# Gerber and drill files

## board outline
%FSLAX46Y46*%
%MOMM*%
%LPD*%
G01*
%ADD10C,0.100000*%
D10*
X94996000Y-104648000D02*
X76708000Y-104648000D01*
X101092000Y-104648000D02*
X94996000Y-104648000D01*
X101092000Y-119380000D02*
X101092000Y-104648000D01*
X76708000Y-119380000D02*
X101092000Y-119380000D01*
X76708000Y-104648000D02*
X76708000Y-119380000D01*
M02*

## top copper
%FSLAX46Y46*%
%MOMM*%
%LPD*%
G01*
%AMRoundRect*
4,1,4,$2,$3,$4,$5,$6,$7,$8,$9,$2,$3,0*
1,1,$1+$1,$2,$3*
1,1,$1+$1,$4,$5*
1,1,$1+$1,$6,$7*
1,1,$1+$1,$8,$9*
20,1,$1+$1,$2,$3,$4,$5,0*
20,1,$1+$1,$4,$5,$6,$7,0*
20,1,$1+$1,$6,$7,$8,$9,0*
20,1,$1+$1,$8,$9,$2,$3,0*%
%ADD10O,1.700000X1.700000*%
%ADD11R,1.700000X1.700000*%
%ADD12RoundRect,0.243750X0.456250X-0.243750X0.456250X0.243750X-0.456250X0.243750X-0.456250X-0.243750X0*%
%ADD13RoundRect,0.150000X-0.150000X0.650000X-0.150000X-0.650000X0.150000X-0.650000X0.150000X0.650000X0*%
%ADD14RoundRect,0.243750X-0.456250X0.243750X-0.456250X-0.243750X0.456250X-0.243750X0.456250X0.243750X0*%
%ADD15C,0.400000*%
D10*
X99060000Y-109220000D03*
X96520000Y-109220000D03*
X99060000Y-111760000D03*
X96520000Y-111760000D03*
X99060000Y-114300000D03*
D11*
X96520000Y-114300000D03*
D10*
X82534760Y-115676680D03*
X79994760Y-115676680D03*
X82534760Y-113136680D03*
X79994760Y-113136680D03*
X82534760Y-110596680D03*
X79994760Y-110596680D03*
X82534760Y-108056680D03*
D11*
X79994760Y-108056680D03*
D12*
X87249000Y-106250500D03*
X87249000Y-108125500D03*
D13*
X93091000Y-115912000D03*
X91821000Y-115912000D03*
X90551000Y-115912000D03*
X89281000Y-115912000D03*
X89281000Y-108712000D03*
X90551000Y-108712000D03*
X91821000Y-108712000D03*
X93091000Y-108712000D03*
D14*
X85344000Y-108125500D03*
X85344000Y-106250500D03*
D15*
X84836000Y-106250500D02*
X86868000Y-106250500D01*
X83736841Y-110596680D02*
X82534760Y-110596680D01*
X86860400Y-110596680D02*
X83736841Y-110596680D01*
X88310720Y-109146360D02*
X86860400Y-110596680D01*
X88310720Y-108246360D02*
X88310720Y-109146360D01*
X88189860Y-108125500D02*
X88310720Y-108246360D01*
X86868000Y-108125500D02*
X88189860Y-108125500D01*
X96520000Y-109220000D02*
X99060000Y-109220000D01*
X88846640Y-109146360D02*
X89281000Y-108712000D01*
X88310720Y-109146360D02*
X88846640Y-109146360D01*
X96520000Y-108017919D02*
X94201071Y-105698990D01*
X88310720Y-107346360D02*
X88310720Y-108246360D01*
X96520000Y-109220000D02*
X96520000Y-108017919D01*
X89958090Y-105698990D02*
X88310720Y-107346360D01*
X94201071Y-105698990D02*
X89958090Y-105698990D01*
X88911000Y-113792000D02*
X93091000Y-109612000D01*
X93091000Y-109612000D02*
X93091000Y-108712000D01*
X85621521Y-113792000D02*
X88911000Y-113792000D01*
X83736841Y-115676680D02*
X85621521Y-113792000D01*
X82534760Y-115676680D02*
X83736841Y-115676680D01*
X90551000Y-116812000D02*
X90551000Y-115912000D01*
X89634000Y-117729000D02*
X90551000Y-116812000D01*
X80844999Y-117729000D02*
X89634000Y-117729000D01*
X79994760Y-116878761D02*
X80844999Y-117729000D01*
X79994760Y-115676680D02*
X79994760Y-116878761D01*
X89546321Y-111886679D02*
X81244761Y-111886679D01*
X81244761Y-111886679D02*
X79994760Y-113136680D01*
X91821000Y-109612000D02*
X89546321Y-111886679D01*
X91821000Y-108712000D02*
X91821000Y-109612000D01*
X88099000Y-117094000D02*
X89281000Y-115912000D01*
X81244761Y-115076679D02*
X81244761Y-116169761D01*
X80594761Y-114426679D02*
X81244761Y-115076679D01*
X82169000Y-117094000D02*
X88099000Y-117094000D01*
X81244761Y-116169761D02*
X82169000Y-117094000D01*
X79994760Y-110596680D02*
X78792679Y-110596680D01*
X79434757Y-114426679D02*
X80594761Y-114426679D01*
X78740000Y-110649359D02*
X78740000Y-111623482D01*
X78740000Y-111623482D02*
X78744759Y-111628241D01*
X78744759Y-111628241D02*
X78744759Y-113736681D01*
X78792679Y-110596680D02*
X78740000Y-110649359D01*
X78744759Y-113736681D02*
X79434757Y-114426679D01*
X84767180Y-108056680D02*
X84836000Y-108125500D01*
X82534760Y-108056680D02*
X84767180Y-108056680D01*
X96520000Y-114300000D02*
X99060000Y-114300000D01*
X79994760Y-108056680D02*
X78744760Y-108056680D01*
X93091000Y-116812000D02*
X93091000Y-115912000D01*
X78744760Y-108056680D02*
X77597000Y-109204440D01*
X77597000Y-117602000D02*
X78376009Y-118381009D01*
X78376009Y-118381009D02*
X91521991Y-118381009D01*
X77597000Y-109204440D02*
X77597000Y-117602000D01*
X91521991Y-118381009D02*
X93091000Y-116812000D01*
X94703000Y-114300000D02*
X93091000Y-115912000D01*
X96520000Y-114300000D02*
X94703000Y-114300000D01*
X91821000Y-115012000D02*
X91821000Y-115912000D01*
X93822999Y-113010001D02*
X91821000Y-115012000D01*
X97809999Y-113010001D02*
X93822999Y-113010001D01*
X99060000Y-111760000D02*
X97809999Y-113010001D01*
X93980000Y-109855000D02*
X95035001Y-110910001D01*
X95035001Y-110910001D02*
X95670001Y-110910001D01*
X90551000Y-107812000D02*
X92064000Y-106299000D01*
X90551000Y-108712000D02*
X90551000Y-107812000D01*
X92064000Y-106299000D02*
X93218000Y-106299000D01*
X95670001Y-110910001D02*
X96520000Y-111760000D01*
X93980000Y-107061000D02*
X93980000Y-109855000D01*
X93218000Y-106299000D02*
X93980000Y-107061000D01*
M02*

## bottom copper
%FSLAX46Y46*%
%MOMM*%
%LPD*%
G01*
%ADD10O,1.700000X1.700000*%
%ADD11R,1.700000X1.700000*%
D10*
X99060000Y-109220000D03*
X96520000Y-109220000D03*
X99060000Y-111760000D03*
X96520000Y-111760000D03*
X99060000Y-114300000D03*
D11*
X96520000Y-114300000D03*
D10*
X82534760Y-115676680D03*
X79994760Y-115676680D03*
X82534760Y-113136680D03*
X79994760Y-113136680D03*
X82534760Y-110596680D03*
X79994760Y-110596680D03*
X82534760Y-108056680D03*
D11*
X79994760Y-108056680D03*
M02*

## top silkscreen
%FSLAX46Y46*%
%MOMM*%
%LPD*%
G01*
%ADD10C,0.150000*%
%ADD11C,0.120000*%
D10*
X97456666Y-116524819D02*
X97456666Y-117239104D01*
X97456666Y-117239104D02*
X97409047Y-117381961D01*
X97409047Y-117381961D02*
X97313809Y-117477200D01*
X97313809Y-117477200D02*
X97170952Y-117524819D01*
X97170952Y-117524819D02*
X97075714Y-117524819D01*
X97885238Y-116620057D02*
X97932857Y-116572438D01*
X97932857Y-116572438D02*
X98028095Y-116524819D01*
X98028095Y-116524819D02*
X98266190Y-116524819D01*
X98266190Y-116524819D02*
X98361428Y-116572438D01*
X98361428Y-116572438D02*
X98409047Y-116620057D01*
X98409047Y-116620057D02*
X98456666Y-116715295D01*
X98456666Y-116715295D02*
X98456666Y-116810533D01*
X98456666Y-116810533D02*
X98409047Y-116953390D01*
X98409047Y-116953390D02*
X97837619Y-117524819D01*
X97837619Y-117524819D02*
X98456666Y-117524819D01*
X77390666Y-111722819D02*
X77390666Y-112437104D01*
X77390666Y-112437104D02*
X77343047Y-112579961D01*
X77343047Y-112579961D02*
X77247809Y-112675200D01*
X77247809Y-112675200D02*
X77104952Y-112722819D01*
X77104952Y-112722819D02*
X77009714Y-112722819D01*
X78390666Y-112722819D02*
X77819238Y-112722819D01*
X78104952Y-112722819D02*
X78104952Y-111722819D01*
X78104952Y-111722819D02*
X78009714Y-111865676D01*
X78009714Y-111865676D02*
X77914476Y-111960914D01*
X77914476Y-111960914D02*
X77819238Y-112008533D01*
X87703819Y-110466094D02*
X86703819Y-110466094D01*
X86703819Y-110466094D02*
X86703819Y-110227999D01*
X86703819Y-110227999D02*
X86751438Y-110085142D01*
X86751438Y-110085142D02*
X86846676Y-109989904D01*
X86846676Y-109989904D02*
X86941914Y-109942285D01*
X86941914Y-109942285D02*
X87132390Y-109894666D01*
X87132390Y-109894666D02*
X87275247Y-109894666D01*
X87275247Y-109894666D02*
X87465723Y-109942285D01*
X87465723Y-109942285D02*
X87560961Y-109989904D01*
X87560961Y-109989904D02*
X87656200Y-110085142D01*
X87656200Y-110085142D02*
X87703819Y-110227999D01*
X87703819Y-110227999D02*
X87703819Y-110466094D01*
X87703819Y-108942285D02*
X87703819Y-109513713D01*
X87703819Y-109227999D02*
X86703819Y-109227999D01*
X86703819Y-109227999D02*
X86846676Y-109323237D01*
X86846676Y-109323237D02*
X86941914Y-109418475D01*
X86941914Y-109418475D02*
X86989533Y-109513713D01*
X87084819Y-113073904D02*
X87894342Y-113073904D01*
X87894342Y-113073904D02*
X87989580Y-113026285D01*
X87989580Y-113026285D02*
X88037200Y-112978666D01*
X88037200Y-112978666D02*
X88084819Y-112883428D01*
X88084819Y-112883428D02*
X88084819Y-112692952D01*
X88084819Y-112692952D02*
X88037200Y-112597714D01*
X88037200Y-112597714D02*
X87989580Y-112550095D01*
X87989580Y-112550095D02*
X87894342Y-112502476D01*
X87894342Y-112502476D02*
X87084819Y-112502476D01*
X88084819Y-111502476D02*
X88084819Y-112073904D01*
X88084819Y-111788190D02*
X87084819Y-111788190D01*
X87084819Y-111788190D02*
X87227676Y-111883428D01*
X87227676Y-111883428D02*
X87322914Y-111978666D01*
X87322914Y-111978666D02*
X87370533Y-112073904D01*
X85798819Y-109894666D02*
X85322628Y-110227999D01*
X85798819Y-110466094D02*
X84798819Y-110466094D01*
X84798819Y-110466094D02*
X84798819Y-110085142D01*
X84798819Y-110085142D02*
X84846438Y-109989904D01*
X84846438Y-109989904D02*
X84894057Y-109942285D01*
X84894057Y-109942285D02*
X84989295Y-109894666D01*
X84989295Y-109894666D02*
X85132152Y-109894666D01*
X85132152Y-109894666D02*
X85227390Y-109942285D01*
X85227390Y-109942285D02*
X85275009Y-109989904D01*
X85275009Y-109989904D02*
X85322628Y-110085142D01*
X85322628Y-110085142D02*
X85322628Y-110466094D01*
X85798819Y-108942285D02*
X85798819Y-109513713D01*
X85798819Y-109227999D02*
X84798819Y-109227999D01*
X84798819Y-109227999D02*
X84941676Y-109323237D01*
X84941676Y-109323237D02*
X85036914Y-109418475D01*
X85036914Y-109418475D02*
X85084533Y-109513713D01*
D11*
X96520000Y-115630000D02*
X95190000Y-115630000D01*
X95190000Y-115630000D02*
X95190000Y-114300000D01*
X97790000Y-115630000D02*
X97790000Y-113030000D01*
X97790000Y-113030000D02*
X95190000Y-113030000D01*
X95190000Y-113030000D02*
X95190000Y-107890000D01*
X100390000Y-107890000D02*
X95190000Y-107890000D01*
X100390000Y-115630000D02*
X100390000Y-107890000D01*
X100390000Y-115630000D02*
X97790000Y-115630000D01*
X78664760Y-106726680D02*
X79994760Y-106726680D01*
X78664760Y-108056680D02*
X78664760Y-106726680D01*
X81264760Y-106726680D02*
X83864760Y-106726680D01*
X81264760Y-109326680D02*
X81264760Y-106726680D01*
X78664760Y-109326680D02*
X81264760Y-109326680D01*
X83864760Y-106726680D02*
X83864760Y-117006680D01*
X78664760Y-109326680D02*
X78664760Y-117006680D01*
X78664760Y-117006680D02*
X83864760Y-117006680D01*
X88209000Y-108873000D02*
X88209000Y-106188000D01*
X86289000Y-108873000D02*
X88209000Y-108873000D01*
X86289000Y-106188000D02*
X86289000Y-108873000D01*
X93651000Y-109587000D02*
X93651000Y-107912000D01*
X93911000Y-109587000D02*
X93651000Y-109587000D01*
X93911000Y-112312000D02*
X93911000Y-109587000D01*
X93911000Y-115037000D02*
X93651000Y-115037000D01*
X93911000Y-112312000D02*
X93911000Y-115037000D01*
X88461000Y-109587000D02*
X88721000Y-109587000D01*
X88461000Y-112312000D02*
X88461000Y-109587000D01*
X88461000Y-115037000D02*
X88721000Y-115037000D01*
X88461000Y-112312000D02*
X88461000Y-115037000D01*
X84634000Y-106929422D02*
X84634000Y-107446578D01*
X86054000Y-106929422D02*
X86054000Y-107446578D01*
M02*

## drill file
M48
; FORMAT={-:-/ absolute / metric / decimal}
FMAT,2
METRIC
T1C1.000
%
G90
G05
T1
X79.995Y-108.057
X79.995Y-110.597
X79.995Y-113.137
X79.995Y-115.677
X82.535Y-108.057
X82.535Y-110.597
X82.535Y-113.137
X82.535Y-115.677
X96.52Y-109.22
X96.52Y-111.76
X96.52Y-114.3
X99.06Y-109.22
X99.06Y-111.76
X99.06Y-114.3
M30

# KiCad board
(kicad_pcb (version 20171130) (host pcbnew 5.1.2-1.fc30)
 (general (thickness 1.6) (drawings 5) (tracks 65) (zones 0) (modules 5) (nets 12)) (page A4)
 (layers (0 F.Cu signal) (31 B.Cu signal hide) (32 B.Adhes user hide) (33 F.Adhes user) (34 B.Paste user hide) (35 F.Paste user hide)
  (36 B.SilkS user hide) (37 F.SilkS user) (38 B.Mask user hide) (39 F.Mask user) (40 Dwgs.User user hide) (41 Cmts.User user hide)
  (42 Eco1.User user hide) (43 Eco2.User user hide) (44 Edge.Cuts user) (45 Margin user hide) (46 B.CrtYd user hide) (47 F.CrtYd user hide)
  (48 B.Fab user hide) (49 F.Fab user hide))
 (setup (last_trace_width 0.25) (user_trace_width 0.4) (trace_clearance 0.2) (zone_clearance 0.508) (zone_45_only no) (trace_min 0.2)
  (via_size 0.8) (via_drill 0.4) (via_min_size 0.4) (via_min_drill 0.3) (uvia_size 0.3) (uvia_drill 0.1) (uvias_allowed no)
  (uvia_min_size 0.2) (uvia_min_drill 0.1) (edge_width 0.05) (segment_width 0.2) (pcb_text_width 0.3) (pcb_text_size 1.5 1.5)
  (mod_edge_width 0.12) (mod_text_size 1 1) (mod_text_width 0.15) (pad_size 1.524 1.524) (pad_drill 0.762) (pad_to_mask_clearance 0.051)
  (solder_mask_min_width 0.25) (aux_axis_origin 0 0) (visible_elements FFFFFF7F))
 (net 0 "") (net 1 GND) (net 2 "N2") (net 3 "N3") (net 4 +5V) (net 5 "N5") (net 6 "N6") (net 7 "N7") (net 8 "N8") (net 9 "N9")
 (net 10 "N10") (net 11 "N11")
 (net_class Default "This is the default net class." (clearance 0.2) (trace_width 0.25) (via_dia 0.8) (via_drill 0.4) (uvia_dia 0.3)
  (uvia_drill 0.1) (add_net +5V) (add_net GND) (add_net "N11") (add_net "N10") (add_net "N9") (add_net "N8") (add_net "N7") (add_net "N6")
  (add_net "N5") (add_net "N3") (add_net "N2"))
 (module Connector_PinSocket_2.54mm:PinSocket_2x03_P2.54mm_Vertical (layer F.Cu) (at 96.52 114.3 180)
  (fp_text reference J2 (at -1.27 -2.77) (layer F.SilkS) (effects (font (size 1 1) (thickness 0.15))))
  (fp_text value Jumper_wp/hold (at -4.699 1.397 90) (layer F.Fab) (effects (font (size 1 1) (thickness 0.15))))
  (fp_line (start 0 -1.33) (end 1.33 -1.33) (layer F.SilkS) (width 0.12))
  (fp_line (start 1.33 -1.33) (end 1.33 0) (layer F.SilkS) (width 0.12))
  (fp_line (start -1.27 -1.33) (end -1.27 1.27) (layer F.SilkS) (width 0.12))
  (fp_line (start -1.27 1.27) (end 1.33 1.27) (layer F.SilkS) (width 0.12))
  (fp_line (start 1.33 1.27) (end 1.33 6.41) (layer F.SilkS) (width 0.12))
  (fp_line (start -3.87 6.41) (end 1.33 6.41) (layer F.SilkS) (width 0.12))
  (fp_line (start -3.87 -1.33) (end -3.87 6.41) (layer F.SilkS) (width 0.12))
  (fp_line (start -3.87 -1.33) (end -1.27 -1.33) (layer F.SilkS) (width 0.12))
  (pad 6 thru_hole oval (at -2.54 5.08 180) (size 1.7 1.7) (drill 1) (layers *.Cu *.Mask) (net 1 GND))
  (pad 5 thru_hole oval (at 0 5.08 180) (size 1.7 1.7) (drill 1) (layers *.Cu *.Mask) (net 1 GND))
  (pad 4 thru_hole oval (at -2.54 2.54 180) (size 1.7 1.7) (drill 1) (layers *.Cu *.Mask) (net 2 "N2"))
  (pad 3 thru_hole oval (at 0 2.54 180) (size 1.7 1.7) (drill 1) (layers *.Cu *.Mask) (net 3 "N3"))
  (pad 2 thru_hole oval (at -2.54 0 180) (size 1.7 1.7) (drill 1) (layers *.Cu *.Mask) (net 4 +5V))
  (pad 1 thru_hole rect (at 0 0 180) (size 1.7 1.7) (drill 1) (layers *.Cu *.Mask) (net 4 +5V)))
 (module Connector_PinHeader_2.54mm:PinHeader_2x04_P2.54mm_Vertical (layer F.Cu) (at 79.99476 108.05668)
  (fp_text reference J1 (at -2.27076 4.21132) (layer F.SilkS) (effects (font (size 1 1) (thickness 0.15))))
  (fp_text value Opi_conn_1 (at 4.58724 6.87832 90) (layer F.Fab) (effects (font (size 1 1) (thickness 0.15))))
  (fp_line (start -1.33 -1.33) (end 0 -1.33) (layer F.SilkS) (width 0.12))
  (fp_line (start -1.33 0) (end -1.33 -1.33) (layer F.SilkS) (width 0.12))
  (fp_line (start 1.27 -1.33) (end 3.87 -1.33) (layer F.SilkS) (width 0.12))
  (fp_line (start 1.27 1.27) (end 1.27 -1.33) (layer F.SilkS) (width 0.12))
  (fp_line (start -1.33 1.27) (end 1.27 1.27) (layer F.SilkS) (width 0.12))
  (fp_line (start 3.87 -1.33) (end 3.87 8.95) (layer F.SilkS) (width 0.12))
  (fp_line (start -1.33 1.27) (end -1.33 8.95) (layer F.SilkS) (width 0.12))
  (fp_line (start -1.33 8.95) (end 3.87 8.95) (layer F.SilkS) (width 0.12))
  (pad 8 thru_hole oval (at 2.54 7.62) (size 1.7 1.7) (drill 1) (layers *.Cu *.Mask) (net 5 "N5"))
  (pad 7 thru_hole oval (at 0 7.62) (size 1.7 1.7) (drill 1) (layers *.Cu *.Mask) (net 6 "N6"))
  (pad 6 thru_hole oval (at 2.54 5.08) (size 1.7 1.7) (drill 1) (layers *.Cu *.Mask) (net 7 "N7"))
  (pad 5 thru_hole oval (at 0 5.08) (size 1.7 1.7) (drill 1) (layers *.Cu *.Mask) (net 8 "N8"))
  (pad 4 thru_hole oval (at 2.54 2.54) (size 1.7 1.7) (drill 1) (layers *.Cu *.Mask) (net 1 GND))
  (pad 3 thru_hole oval (at 0 2.54) (size 1.7 1.7) (drill 1) (layers *.Cu *.Mask) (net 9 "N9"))
  (pad 2 thru_hole oval (at 2.54 0) (size 1.7 1.7) (drill 1) (layers *.Cu *.Mask) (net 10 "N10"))
  (pad 1 thru_hole rect (at 0 0) (size 1.7 1.7) (drill 1) (layers *.Cu *.Mask) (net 4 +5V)))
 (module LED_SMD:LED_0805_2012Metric (layer F.Cu) (at 87.249 107.188 90)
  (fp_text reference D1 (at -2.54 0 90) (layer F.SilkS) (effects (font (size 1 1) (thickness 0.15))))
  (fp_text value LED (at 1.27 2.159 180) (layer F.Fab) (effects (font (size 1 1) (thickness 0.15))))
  (fp_line (start -1.685 0.96) (end 1 0.96) (layer F.SilkS) (width 0.12))
  (fp_line (start -1.685 -0.96) (end -1.685 0.96) (layer F.SilkS) (width 0.12))
  (fp_line (start 1 -0.96) (end -1.685 -0.96) (layer F.SilkS) (width 0.12))
  (pad 2 smd roundrect (at 0.9375 0 90) (size 0.975 1.4) (layers F.Cu F.Paste F.Mask) (roundrect_rratio 0.25) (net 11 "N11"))
  (pad 1 smd roundrect (at -0.9375 0 90) (size 0.975 1.4) (layers F.Cu F.Paste F.Mask) (roundrect_rratio 0.25) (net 1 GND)))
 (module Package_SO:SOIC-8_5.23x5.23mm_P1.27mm (layer F.Cu) (at 91.186 112.312 270)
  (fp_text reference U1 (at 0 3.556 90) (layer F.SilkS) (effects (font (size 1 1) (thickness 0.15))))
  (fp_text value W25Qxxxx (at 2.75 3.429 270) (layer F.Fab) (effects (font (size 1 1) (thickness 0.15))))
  (fp_line (start -2.725 -2.465) (end -4.4 -2.465) (layer F.SilkS) (width 0.12))
  (fp_line (start -2.725 -2.725) (end -2.725 -2.465) (layer F.SilkS) (width 0.12))
  (fp_line (start 0 -2.725) (end -2.725 -2.725) (layer F.SilkS) (width 0.12))
  (fp_line (start 2.725 -2.725) (end 2.725 -2.465) (layer F.SilkS) (width 0.12))
  (fp_line (start 0 -2.725) (end 2.725 -2.725) (layer F.SilkS) (width 0.12))
  (fp_line (start -2.725 2.725) (end -2.725 2.465) (layer F.SilkS) (width 0.12))
  (fp_line (start 0 2.725) (end -2.725 2.725) (layer F.SilkS) (width 0.12))
  (fp_line (start 2.725 2.725) (end 2.725 2.465) (layer F.SilkS) (width 0.12))
  (fp_line (start 0 2.725) (end 2.725 2.725) (layer F.SilkS) (width 0.12))
  (pad 8 smd roundrect (at 3.6 -1.905 270) (size 1.6 0.6) (layers F.Cu F.Paste F.Mask) (roundrect_rratio 0.25) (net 4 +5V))
  (pad 7 smd roundrect (at 3.6 -0.635 270) (size 1.6 0.6) (layers F.Cu F.Paste F.Mask) (roundrect_rratio 0.25) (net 2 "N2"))
  (pad 6 smd roundrect (at 3.6 0.635 270) (size 1.6 0.6) (layers F.Cu F.Paste F.Mask) (roundrect_rratio 0.25) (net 6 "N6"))
  (pad 5 smd roundrect (at 3.6 1.905 270) (size 1.6 0.6) (layers F.Cu F.Paste F.Mask) (roundrect_rratio 0.25) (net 9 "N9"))
  (pad 4 smd roundrect (at -3.6 1.905 270) (size 1.6 0.6) (layers F.Cu F.Paste F.Mask) (roundrect_rratio 0.25) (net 1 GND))
  (pad 3 smd roundrect (at -3.6 0.635 270) (size 1.6 0.6) (layers F.Cu F.Paste F.Mask) (roundrect_rratio 0.25) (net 3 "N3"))
  (pad 2 smd roundrect (at -3.6 -0.635 270) (size 1.6 0.6) (layers F.Cu F.Paste F.Mask) (roundrect_rratio 0.25) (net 8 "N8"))
  (pad 1 smd roundrect (at -3.6 -1.905 270) (size 1.6 0.6) (layers F.Cu F.Paste F.Mask) (roundrect_rratio 0.25) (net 5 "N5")))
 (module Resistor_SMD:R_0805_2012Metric (layer F.Cu) (at 85.344 107.188 270)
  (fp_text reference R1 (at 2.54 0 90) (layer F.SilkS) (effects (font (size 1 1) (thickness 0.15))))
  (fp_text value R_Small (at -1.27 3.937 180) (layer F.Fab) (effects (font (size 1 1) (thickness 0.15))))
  (fp_line (start -0.258578 0.71) (end 0.258578 0.71) (layer F.SilkS) (width 0.12))
  (fp_line (start -0.258578 -0.71) (end 0.258578 -0.71) (layer F.SilkS) (width 0.12))
  (pad 2 smd roundrect (at 0.9375 0 270) (size 0.975 1.4) (layers F.Cu F.Paste F.Mask) (roundrect_rratio 0.25) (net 10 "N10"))
  (pad 1 smd roundrect (at -0.9375 0 270) (size 0.975 1.4) (layers F.Cu F.Paste F.Mask) (roundrect_rratio 0.25) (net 11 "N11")))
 (gr_line (start 94.996 104.648) (end 76.708 104.648) (layer Edge.Cuts) (width 0.1))
 (gr_line (start 101.092 104.648) (end 94.996 104.648) (layer Edge.Cuts) (width 0.1))
 (gr_line (start 101.092 119.38) (end 101.092 104.648) (layer Edge.Cuts) (width 0.1))
 (gr_line (start 76.708 119.38) (end 101.092 119.38) (layer Edge.Cuts) (width 0.1))
 (gr_line (start 76.708 104.648) (end 76.708 119.38) (layer Edge.Cuts) (width 0.1))
 (segment (start 84.836 106.2505) (end 86.868 106.2505) (width 0.4) (layer F.Cu) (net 11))
 (segment (start 83.736841 110.59668) (end 82.53476 110.59668) (width 0.4) (layer F.Cu) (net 1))
 (segment (start 86.8604 110.59668) (end 83.736841 110.59668) (width 0.4) (layer F.Cu) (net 1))
 (segment (start 88.31072 109.14636) (end 86.8604 110.59668) (width 0.4) (layer F.Cu) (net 1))
 (segment (start 88.31072 108.24636) (end 88.31072 109.14636) (width 0.4) (layer F.Cu) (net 1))
 (segment (start 88.18986 108.1255) (end 88.31072 108.24636) (width 0.4) (layer F.Cu) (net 1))
 (segment (start 86.868 108.1255) (end 88.18986 108.1255) (width 0.4) (layer F.Cu) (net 1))
 (segment (start 96.52 109.22) (end 99.06 109.22) (width 0.4) (layer F.Cu) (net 1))
 (segment (start 88.84664 109.14636) (end 89.281 108.712) (width 0.4) (layer F.Cu) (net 1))
 (segment (start 88.31072 109.14636) (end 88.84664 109.14636) (width 0.4) (layer F.Cu) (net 1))
 (segment (start 96.52 108.017919) (end 94.201071 105.69899) (width 0.4) (layer F.Cu) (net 1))
 (segment (start 88.31072 107.34636) (end 88.31072 108.24636) (width 0.4) (layer F.Cu) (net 1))
 (segment (start 96.52 109.22) (end 96.52 108.017919) (width 0.4) (layer F.Cu) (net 1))
 (segment (start 89.95809 105.69899) (end 88.31072 107.34636) (width 0.4) (layer F.Cu) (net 1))
 (segment (start 94.201071 105.69899) (end 89.95809 105.69899) (width 0.4) (layer F.Cu) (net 1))
 (segment (start 88.911 113.792) (end 93.091 109.612) (width 0.4) (layer F.Cu) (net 5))
 (segment (start 93.091 109.612) (end 93.091 108.712) (width 0.4) (layer F.Cu) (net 5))
 (segment (start 85.621521 113.792) (end 88.911 113.792) (width 0.4) (layer F.Cu) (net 5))
 (segment (start 83.736841 115.67668) (end 85.621521 113.792) (width 0.4) (layer F.Cu) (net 5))
 (segment (start 82.53476 115.67668) (end 83.736841 115.67668) (width 0.4) (layer F.Cu) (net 5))
 (segment (start 90.551 116.812) (end 90.551 115.912) (width 0.4) (layer F.Cu) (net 6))
 (segment (start 89.634 117.729) (end 90.551 116.812) (width 0.4) (layer F.Cu) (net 6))
 (segment (start 80.844999 117.729) (end 89.634 117.729) (width 0.4) (layer F.Cu) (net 6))
 (segment (start 79.99476 116.878761) (end 80.844999 117.729) (width 0.4) (layer F.Cu) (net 6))
 (segment (start 79.99476 115.67668) (end 79.99476 116.878761) (width 0.4) (layer F.Cu) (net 6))
 (segment (start 89.546321 111.886679) (end 81.244761 111.886679) (width 0.4) (layer F.Cu) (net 8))
 (segment (start 81.244761 111.886679) (end 79.99476 113.13668) (width 0.4) (layer F.Cu) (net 8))
 (segment (start 91.821 109.612) (end 89.546321 111.886679) (width 0.4) (layer F.Cu) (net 8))
 (segment (start 91.821 108.712) (end 91.821 109.612) (width 0.4) (layer F.Cu) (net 8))
 (segment (start 88.099 117.094) (end 89.281 115.912) (width 0.4) (layer F.Cu) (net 9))
 (segment (start 81.244761 115.076679) (end 81.244761 116.169761) (width 0.4) (layer F.Cu) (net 9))
 (segment (start 80.594761 114.426679) (end 81.244761 115.076679) (width 0.4) (layer F.Cu) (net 9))
 (segment (start 82.169 117.094) (end 88.099 117.094) (width 0.4) (layer F.Cu) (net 9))
 (segment (start 81.244761 116.169761) (end 82.169 117.094) (width 0.4) (layer F.Cu) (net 9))
 (segment (start 79.99476 110.59668) (end 78.792679 110.59668) (width 0.4) (layer F.Cu) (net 9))
 (segment (start 79.434757 114.426679) (end 80.594761 114.426679) (width 0.4) (layer F.Cu) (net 9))
 (segment (start 78.74 110.649359) (end 78.74 111.623482) (width 0.4) (layer F.Cu) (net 9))
 (segment (start 78.74 111.623482) (end 78.744759 111.628241) (width 0.4) (layer F.Cu) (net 9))
 (segment (start 78.744759 111.628241) (end 78.744759 113.736681) (width 0.4) (layer F.Cu) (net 9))
 (segment (start 78.792679 110.59668) (end 78.74 110.649359) (width 0.4) (layer F.Cu) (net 9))
 (segment (start 78.744759 113.736681) (end 79.434757 114.426679) (width 0.4) (layer F.Cu) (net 9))
 (segment (start 84.76718 108.05668) (end 84.836 108.1255) (width 0.4) (layer F.Cu) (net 10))
 (segment (start 82.53476 108.05668) (end 84.76718 108.05668) (width 0.4) (layer F.Cu) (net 10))
 (segment (start 96.52 114.3) (end 99.06 114.3) (width 0.4) (layer F.Cu) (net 4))
 (segment (start 79.99476 108.05668) (end 78.74476 108.05668) (width 0.4) (layer F.Cu) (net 4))
 (segment (start 93.091 116.812) (end 93.091 115.912) (width 0.4) (layer F.Cu) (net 4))
 (segment (start 78.74476 108.05668) (end 77.597 109.20444) (width 0.4) (layer F.Cu) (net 4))
 (segment (start 77.597 117.602) (end 78.376009 118.381009) (width 0.4) (layer F.Cu) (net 4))
 (segment (start 78.376009 118.381009) (end 91.521991 118.381009) (width 0.4) (layer F.Cu) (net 4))
 (segment (start 77.597 109.20444) (end 77.597 117.602) (width 0.4) (layer F.Cu) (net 4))
 (segment (start 91.521991 118.381009) (end 93.091 116.812) (width 0.4) (layer F.Cu) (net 4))
 (segment (start 94.703 114.3) (end 93.091 115.912) (width 0.4) (layer F.Cu) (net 4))
 (segment (start 96.52 114.3) (end 94.703 114.3) (width 0.4) (layer F.Cu) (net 4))
 (segment (start 91.821 115.012) (end 91.821 115.912) (width 0.4) (layer F.Cu) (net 2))
 (segment (start 93.822999 113.010001) (end 91.821 115.012) (width 0.4) (layer F.Cu) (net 2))
 (segment (start 97.809999 113.010001) (end 93.822999 113.010001) (width 0.4) (layer F.Cu) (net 2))
 (segment (start 99.06 111.76) (end 97.809999 113.010001) (width 0.4) (layer F.Cu) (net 2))
 (segment (start 93.98 109.855) (end 95.035001 110.910001) (width 0.4) (layer F.Cu) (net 3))
 (segment (start 95.035001 110.910001) (end 95.670001 110.910001) (width 0.4) (layer F.Cu) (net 3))
 (segment (start 90.551 107.812) (end 92.064 106.299) (width 0.4) (layer F.Cu) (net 3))
 (segment (start 90.551 108.712) (end 90.551 107.812) (width 0.4) (layer F.Cu) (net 3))
 (segment (start 92.064 106.299) (end 93.218 106.299) (width 0.4) (layer F.Cu) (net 3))
 (segment (start 95.670001 110.910001) (end 96.52 111.76) (width 0.4) (layer F.Cu) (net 3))
 (segment (start 93.98 107.061) (end 93.98 109.855) (width 0.4) (layer F.Cu) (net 3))
 (segment (start 93.218 106.299) (end 93.98 107.061) (width 0.4) (layer F.Cu) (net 3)))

